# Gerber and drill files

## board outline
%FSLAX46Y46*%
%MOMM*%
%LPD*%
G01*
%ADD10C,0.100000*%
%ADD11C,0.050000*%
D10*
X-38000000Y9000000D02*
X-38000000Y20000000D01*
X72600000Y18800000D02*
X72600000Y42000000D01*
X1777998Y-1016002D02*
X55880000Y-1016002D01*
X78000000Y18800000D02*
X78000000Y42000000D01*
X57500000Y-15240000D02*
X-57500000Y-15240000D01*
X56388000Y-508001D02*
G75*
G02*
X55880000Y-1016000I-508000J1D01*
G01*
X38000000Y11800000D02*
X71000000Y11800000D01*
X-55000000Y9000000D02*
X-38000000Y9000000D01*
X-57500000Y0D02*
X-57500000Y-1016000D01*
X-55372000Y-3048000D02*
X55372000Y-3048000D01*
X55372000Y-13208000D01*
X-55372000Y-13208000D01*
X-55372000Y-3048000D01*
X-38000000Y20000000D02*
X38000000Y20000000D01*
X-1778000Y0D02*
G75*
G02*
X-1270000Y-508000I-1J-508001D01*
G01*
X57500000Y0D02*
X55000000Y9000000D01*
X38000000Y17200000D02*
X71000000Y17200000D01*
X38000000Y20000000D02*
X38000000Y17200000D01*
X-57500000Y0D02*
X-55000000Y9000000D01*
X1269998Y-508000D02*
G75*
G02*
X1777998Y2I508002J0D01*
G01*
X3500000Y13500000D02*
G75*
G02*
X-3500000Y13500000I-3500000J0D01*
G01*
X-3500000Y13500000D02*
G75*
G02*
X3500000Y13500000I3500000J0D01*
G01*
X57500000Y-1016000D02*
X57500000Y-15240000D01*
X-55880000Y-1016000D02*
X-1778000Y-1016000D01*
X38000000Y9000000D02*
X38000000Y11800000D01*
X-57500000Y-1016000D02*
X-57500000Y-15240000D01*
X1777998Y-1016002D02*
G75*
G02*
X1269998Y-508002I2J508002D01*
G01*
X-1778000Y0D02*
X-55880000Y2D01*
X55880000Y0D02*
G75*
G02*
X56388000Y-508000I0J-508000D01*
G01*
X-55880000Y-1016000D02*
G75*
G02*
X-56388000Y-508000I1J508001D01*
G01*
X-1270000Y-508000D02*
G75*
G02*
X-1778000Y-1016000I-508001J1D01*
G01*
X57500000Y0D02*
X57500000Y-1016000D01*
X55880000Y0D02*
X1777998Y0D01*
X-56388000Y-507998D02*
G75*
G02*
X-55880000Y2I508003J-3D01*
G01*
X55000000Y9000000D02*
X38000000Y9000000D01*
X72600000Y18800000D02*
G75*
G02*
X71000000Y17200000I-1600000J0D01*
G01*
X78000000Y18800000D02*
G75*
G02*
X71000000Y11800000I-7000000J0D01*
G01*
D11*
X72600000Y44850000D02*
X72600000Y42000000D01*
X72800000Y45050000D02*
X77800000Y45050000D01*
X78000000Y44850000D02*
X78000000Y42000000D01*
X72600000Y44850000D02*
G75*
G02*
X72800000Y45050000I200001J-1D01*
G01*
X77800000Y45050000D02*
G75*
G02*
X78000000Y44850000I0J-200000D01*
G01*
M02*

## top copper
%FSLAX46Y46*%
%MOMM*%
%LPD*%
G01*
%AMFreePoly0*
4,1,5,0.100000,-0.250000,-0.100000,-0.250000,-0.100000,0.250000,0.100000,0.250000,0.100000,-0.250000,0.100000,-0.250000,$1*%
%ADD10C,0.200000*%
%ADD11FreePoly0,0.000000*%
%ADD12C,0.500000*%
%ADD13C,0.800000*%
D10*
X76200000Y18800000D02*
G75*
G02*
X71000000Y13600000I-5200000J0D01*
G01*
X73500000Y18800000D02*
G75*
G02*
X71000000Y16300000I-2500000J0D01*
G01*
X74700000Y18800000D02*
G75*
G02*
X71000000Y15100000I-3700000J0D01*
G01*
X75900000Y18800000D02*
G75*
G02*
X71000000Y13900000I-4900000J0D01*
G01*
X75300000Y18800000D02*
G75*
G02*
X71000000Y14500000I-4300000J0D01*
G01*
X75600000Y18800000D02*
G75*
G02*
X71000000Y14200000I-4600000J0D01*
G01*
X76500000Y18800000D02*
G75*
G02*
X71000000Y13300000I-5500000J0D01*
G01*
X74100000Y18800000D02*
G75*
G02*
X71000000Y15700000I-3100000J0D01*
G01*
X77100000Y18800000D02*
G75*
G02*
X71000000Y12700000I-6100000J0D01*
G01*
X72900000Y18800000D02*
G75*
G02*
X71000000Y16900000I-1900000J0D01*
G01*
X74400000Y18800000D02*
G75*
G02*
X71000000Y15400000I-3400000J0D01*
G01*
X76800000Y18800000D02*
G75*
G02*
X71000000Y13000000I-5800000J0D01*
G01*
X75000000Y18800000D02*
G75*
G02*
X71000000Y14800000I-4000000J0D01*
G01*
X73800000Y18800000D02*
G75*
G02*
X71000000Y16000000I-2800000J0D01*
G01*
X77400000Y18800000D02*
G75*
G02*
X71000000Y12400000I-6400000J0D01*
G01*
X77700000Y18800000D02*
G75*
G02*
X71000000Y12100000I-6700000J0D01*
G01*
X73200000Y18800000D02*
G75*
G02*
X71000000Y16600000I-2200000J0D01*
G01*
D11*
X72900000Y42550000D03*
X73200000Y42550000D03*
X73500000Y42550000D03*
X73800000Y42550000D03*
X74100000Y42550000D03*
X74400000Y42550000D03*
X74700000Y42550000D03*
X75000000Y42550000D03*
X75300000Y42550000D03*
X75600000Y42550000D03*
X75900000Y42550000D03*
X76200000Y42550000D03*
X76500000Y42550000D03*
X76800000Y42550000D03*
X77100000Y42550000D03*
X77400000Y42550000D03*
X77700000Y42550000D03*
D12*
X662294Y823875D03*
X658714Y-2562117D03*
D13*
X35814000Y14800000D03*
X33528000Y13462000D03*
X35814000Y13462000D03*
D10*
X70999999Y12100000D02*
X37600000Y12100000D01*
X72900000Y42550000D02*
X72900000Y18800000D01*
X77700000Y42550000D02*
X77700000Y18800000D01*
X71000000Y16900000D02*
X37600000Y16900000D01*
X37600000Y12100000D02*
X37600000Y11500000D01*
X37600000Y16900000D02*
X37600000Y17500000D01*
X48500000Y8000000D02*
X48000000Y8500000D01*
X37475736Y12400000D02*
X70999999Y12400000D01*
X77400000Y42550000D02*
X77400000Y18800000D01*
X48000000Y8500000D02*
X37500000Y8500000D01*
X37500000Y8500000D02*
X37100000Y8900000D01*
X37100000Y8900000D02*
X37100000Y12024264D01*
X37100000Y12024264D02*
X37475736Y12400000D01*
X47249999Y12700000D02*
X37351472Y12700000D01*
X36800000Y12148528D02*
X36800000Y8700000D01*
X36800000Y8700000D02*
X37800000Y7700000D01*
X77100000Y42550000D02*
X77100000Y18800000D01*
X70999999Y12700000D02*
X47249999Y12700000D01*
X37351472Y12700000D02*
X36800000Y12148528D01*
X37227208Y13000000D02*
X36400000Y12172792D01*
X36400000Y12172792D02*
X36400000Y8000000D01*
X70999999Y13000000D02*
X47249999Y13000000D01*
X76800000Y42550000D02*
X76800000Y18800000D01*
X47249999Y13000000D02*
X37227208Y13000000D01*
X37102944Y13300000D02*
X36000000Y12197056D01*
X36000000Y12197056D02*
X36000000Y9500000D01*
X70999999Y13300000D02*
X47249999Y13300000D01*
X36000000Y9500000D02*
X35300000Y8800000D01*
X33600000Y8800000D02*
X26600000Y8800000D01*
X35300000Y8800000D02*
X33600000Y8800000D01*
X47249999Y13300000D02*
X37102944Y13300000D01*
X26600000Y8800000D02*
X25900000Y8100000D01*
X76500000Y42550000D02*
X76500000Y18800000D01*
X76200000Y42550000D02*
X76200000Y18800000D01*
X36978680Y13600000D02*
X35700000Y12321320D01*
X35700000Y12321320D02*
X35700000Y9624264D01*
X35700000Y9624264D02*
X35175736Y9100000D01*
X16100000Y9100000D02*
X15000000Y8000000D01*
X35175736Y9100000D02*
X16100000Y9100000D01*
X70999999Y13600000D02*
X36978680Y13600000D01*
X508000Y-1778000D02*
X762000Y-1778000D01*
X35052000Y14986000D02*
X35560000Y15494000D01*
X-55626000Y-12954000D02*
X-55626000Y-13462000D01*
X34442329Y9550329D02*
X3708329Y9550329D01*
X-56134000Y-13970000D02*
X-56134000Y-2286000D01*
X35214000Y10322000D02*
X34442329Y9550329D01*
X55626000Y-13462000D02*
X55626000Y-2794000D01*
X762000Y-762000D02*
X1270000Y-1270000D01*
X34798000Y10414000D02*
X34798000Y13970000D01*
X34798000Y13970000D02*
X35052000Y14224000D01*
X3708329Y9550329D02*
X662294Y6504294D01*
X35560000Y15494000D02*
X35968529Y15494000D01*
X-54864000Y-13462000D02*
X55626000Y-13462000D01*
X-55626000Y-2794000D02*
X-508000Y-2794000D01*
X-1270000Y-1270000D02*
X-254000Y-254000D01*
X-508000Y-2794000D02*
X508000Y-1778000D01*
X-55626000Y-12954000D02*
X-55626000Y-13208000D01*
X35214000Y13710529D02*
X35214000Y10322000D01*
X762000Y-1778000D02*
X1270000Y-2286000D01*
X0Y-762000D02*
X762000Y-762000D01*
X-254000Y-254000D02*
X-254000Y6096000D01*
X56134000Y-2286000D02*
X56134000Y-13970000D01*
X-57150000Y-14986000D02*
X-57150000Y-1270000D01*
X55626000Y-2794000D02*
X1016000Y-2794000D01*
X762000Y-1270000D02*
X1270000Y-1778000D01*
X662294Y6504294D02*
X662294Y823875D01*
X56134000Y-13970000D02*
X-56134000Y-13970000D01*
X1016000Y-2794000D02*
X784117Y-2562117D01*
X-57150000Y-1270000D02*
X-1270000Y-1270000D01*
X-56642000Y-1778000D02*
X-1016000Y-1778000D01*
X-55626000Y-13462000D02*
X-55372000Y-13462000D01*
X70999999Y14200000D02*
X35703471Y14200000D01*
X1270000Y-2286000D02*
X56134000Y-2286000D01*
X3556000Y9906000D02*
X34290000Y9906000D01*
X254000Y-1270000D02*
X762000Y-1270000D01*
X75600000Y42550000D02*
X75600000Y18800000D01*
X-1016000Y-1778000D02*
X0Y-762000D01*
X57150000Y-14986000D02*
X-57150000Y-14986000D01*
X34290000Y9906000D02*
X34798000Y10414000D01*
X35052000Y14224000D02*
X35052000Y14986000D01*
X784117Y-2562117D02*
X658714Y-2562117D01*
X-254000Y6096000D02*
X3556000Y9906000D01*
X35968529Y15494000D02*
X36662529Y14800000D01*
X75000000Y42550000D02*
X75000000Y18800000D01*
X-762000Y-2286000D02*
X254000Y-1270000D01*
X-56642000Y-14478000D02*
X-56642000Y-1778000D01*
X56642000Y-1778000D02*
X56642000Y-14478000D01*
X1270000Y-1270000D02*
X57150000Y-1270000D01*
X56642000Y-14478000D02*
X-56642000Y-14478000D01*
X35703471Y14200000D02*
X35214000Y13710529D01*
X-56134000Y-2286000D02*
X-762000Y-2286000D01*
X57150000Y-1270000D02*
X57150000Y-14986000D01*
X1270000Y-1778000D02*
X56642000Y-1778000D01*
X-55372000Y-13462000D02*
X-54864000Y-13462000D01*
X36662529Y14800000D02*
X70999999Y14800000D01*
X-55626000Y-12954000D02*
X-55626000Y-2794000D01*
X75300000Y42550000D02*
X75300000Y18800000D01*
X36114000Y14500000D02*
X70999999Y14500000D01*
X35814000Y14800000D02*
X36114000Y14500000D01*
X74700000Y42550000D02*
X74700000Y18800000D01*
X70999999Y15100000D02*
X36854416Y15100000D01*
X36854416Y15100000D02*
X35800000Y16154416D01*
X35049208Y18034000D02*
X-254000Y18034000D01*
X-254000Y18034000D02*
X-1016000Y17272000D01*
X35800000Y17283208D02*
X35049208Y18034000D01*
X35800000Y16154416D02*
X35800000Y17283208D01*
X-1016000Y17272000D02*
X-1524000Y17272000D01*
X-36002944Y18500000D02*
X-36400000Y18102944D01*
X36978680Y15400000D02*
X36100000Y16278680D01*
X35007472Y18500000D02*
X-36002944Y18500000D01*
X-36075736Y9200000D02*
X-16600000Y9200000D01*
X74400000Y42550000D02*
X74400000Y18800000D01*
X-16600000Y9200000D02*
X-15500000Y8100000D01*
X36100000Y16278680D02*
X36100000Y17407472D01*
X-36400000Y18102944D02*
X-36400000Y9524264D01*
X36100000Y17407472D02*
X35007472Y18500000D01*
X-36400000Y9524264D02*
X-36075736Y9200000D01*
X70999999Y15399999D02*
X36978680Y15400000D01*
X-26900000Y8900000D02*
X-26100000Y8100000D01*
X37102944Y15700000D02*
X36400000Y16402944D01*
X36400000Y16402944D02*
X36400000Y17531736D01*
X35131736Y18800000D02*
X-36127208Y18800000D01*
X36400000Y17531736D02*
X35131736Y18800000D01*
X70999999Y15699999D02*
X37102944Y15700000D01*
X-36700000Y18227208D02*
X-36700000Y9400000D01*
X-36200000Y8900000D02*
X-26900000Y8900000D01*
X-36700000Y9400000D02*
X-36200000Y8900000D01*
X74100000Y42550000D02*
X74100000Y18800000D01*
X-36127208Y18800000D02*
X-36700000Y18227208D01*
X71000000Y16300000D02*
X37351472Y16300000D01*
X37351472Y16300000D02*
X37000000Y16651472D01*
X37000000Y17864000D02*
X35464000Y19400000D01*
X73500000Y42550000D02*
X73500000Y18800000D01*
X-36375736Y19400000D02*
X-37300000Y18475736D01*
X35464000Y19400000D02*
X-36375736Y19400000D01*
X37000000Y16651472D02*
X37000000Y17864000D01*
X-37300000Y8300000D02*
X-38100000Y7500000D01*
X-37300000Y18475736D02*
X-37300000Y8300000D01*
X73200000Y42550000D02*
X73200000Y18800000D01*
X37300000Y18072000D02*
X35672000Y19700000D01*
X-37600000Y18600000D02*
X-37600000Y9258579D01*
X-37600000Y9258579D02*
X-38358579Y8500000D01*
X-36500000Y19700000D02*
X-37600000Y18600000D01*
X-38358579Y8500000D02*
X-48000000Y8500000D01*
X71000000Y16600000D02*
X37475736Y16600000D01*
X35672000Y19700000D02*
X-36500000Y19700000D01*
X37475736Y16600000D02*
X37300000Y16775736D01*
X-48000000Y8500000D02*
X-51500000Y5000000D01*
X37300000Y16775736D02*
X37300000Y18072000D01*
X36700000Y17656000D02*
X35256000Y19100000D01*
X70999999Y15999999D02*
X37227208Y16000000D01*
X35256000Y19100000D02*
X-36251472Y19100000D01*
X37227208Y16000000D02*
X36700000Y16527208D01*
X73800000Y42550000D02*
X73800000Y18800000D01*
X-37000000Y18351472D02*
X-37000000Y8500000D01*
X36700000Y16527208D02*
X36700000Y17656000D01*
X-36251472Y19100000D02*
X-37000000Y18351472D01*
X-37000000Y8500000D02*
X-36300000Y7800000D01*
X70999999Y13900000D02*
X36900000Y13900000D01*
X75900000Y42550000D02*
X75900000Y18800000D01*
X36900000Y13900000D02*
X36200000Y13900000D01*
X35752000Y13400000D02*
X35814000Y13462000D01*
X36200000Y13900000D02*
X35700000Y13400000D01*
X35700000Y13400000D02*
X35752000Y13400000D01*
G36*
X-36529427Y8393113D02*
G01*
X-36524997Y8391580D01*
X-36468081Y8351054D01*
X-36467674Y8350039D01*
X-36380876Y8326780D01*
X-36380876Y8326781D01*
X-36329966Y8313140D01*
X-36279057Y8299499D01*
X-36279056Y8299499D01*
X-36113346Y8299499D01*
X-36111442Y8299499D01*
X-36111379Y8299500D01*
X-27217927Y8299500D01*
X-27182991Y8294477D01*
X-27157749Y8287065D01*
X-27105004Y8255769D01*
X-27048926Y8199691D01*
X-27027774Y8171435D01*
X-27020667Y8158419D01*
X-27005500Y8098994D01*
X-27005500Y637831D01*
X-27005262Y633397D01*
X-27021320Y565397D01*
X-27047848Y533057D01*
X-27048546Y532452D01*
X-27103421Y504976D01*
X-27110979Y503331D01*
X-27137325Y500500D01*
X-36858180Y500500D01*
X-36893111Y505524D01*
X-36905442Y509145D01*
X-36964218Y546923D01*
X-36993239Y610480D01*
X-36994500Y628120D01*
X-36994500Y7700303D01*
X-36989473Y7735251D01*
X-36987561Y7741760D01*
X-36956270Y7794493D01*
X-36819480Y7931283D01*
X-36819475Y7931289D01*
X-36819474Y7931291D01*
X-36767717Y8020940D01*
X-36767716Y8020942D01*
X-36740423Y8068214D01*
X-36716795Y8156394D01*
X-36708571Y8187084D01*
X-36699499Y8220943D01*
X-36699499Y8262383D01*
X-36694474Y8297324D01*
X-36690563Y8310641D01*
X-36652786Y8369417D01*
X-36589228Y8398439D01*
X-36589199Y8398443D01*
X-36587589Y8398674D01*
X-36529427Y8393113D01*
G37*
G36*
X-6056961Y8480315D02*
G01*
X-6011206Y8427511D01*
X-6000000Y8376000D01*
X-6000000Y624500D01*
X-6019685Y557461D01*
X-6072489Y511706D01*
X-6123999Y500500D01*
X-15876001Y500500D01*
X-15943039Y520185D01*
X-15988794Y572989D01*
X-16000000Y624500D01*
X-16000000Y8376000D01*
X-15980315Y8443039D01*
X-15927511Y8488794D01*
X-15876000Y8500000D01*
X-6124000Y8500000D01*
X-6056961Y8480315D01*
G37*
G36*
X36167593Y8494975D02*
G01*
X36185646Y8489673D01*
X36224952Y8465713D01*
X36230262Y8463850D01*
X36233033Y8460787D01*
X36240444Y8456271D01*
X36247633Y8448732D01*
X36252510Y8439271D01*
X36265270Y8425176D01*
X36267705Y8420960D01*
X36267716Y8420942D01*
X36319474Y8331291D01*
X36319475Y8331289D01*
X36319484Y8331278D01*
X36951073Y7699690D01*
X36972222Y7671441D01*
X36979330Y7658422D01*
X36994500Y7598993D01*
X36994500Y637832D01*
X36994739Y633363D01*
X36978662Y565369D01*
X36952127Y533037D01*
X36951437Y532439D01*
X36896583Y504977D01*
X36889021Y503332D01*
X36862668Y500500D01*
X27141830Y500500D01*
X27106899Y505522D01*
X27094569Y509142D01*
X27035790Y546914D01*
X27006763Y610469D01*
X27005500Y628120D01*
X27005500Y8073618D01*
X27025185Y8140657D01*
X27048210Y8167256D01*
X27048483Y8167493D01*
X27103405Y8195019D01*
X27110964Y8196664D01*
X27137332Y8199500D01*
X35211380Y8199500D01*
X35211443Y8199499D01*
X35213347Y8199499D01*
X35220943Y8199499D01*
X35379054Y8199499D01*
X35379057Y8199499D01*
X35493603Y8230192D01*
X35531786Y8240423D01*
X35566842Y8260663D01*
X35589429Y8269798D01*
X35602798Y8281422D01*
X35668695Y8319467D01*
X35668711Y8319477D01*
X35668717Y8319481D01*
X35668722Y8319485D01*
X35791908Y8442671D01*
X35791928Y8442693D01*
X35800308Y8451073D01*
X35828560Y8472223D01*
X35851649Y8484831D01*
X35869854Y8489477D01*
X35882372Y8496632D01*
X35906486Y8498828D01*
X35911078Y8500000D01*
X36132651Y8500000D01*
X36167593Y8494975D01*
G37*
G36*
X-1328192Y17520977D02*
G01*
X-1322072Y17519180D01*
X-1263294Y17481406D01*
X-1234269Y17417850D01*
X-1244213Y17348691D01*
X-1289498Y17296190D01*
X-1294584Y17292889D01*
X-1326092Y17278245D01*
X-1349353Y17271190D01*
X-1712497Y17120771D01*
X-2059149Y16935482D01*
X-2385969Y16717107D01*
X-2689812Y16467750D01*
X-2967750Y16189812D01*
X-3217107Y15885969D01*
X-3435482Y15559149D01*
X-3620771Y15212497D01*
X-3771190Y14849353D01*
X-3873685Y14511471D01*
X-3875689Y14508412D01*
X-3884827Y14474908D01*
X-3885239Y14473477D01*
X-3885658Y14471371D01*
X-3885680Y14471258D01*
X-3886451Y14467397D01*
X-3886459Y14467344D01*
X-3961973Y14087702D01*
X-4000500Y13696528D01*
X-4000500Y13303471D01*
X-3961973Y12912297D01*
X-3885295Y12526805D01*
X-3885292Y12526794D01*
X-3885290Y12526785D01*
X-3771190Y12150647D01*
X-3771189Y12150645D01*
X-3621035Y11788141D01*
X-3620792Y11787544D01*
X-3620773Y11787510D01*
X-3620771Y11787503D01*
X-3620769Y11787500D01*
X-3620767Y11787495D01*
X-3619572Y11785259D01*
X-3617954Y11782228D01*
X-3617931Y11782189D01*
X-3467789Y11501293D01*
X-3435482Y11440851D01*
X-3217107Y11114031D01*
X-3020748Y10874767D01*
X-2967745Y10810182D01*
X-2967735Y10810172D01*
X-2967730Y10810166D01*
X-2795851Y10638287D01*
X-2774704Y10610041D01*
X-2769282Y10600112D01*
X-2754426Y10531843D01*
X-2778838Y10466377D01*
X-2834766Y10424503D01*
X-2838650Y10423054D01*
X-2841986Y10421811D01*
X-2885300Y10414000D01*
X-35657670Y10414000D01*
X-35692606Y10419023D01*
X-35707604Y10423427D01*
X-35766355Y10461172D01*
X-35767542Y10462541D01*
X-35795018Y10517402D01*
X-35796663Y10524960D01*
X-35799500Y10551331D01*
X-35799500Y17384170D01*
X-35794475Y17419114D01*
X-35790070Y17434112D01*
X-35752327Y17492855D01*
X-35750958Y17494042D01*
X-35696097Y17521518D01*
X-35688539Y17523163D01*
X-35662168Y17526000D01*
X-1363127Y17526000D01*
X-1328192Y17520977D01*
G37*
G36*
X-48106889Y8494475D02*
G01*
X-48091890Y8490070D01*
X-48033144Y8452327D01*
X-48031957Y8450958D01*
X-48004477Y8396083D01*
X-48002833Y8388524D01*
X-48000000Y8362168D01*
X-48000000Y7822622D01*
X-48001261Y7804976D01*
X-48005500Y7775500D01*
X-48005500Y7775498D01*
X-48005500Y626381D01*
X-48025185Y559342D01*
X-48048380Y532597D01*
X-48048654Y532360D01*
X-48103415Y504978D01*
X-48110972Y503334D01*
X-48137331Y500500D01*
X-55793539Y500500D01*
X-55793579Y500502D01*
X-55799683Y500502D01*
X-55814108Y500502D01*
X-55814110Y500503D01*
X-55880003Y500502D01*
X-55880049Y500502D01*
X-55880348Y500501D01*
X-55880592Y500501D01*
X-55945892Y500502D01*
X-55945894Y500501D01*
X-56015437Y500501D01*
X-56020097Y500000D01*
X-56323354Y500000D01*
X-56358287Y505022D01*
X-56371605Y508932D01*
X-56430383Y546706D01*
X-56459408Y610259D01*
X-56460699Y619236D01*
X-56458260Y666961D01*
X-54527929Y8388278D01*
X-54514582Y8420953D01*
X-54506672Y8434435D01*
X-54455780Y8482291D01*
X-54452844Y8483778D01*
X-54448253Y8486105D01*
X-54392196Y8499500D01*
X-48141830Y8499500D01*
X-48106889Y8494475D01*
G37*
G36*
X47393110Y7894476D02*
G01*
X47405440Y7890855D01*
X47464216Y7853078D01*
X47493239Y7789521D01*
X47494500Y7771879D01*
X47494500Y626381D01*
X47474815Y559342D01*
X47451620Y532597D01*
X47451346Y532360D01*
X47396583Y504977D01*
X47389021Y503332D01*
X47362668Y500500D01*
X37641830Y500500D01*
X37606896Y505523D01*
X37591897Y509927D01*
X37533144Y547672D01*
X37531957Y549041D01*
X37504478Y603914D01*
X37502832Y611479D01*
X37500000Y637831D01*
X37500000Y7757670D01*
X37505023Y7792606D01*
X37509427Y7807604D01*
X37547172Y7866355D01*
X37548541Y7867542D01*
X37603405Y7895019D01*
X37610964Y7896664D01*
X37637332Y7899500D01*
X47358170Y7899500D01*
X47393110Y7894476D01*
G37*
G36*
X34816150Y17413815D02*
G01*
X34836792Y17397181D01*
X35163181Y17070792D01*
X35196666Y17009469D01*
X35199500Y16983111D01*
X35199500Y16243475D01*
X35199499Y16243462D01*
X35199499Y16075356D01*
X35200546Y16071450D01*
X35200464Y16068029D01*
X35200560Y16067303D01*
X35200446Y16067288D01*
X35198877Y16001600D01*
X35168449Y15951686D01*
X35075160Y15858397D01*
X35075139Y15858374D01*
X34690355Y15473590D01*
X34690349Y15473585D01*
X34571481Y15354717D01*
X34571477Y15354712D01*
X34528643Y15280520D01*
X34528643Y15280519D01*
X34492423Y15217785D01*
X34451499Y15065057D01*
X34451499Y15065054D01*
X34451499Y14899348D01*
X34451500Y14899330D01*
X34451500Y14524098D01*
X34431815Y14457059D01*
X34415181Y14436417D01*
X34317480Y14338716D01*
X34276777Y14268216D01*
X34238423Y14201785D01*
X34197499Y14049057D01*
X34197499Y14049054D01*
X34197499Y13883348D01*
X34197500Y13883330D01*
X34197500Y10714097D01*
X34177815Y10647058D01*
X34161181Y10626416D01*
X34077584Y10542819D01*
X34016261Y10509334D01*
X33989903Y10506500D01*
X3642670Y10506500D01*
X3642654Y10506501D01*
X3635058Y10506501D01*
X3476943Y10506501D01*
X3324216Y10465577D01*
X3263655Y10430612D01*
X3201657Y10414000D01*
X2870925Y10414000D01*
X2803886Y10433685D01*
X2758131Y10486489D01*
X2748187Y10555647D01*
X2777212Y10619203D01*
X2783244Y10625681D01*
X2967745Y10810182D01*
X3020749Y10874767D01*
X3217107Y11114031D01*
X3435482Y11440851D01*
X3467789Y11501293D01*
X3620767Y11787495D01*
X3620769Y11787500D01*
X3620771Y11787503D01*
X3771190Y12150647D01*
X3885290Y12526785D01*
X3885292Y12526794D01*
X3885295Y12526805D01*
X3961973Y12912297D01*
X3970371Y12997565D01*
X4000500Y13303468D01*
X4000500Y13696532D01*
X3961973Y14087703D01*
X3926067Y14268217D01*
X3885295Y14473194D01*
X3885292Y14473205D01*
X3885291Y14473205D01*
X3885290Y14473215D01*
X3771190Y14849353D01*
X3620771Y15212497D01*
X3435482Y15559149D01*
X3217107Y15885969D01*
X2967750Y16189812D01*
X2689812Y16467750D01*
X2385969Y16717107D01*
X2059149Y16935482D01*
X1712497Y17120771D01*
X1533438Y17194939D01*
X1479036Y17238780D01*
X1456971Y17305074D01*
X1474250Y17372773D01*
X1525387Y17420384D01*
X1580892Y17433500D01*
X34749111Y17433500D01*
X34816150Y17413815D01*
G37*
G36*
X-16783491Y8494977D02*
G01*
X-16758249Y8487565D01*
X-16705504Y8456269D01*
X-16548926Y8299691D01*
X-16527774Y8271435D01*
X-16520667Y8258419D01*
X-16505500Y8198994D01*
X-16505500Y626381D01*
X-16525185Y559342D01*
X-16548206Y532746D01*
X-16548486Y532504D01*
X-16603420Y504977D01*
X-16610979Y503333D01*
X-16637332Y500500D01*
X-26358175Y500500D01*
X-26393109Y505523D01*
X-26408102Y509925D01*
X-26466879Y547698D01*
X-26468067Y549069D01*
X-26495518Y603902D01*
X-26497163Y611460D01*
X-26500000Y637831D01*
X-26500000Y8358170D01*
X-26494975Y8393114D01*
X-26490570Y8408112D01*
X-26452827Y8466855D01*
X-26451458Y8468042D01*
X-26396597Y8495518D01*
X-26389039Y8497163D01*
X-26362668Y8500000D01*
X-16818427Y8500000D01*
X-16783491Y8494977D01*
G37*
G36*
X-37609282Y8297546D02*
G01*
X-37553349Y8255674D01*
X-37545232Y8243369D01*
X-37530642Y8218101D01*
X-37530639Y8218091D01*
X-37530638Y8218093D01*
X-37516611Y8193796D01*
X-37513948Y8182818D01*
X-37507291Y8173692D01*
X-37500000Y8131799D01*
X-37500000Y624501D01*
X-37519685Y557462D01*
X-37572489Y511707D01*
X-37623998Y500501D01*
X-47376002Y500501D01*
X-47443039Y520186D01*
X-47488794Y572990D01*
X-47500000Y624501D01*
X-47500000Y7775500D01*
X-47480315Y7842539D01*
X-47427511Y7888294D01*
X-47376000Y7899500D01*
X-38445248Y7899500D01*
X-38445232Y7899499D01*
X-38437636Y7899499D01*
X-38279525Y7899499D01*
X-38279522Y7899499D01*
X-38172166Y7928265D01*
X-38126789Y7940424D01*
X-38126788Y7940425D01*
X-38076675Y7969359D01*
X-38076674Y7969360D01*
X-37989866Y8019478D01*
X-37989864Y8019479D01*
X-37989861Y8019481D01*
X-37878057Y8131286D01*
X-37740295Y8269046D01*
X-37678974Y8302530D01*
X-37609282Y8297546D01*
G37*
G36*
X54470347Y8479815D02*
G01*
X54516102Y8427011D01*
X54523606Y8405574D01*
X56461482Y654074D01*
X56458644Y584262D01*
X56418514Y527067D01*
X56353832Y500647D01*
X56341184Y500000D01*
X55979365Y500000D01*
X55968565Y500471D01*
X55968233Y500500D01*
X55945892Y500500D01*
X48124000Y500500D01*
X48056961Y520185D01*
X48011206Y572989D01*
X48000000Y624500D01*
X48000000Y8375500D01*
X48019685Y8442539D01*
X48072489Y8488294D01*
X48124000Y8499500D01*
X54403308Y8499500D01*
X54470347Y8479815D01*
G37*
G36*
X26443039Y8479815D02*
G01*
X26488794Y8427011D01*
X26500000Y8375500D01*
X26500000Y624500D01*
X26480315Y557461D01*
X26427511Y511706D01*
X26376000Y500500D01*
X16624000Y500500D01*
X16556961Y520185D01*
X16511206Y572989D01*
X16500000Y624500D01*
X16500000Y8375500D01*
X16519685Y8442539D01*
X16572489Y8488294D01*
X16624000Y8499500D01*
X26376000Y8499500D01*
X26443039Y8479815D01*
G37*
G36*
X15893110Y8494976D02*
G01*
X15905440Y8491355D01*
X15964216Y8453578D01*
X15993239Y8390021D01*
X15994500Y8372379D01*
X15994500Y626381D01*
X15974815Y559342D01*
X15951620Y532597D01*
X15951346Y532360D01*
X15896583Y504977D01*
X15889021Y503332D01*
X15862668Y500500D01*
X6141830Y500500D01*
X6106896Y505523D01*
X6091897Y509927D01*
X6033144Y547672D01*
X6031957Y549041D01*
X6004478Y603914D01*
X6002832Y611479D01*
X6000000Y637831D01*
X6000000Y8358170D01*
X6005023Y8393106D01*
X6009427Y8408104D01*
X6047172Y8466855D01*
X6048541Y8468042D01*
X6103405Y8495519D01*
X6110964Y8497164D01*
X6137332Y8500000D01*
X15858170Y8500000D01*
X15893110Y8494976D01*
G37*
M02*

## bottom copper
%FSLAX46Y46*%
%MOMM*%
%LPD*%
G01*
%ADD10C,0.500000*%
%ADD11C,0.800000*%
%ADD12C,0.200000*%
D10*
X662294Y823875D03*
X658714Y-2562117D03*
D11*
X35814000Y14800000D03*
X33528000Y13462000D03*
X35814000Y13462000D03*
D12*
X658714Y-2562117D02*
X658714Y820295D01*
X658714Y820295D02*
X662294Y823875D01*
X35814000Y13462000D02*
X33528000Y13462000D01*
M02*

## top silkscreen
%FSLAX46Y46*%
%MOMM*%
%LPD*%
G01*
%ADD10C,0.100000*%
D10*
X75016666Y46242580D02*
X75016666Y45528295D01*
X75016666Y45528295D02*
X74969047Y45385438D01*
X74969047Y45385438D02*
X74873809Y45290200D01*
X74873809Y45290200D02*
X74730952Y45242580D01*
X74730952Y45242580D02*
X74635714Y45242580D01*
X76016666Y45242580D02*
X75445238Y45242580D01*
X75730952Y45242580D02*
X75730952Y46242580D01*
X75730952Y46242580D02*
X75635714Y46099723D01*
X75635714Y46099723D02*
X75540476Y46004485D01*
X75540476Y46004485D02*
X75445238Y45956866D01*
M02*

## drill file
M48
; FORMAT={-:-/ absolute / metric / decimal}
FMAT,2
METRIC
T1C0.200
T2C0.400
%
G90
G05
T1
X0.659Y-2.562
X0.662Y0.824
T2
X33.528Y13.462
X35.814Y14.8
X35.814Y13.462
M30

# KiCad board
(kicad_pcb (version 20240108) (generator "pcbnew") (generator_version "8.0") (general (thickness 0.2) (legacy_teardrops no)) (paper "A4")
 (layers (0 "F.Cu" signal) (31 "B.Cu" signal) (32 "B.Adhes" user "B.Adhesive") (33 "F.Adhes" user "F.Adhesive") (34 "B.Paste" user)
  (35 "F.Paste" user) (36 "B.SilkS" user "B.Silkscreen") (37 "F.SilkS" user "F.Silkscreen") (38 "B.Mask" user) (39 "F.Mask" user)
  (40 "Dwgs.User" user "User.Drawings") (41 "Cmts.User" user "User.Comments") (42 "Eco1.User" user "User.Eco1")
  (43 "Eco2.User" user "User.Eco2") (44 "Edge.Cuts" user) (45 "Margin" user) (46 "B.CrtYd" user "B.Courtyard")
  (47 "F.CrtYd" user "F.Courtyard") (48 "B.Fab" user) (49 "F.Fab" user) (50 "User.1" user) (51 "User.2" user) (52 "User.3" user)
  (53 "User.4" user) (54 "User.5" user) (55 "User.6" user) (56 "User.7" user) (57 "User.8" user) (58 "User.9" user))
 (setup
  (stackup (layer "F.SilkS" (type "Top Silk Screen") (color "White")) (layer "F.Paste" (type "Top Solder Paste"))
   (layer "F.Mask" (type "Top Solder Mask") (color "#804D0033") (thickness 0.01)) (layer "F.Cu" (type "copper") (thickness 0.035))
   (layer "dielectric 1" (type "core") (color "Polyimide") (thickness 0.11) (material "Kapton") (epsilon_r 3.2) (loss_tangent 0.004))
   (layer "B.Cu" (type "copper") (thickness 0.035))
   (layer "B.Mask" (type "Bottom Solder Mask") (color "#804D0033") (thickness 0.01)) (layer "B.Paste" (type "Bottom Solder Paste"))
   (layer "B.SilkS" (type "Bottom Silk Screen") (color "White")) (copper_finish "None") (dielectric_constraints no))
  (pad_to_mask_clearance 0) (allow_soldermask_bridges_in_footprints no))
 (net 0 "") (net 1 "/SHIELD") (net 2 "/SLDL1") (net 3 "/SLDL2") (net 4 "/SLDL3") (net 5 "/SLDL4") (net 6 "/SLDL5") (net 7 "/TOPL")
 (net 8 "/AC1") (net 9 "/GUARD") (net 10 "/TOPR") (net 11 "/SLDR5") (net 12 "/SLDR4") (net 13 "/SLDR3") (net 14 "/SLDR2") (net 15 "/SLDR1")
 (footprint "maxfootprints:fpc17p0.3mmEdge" (layer "F.Cu") (at 75.3 -45.05)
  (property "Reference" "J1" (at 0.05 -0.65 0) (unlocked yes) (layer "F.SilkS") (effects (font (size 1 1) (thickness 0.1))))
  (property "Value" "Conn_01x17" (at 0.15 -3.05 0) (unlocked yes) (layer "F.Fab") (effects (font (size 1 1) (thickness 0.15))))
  (fp_line (start -2.7 0.2) (end -2.7 3.05) (stroke (width 0.05) (type default)) (layer "Edge.Cuts"))
  (fp_line (start -2.5 0) (end 2.5 0) (stroke (width 0.05) (type default)) (layer "Edge.Cuts"))
  (fp_line (start 2.7 0.2) (end 2.7 3.05) (stroke (width 0.05) (type default)) (layer "Edge.Cuts"))
  (fp_arc (start -2.7 0.2) (mid -2.641421 0.058579) (end -2.5 0) (stroke (width 0.05) (type default)) (layer "Edge.Cuts"))
  (fp_arc (start 2.5 0) (mid 2.641421 0.058579) (end 2.7 0.2) (stroke (width 0.05) (type default)) (layer "Edge.Cuts"))
  (pad "1" connect custom (at -2.4 2.5) (size 0.2 0.5) (layers "F.Cu") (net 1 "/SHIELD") (options (clearance outline) (anchor rect))
   (primitives))
  (pad "2" connect custom (at -2.1 2.5) (size 0.2 0.5) (layers "F.Cu") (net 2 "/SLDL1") (options (clearance outline) (anchor rect))
   (primitives))
  (pad "3" connect custom (at -1.8 2.5) (size 0.2 0.5) (layers "F.Cu") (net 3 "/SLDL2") (options (clearance outline) (anchor rect))
   (primitives))
  (pad "4" connect custom (at -1.5 2.5) (size 0.2 0.5) (layers "F.Cu") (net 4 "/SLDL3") (options (clearance outline) (anchor rect))
   (primitives))
  (pad "5" connect custom (at -1.2 2.5) (size 0.2 0.5) (layers "F.Cu") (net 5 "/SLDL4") (options (clearance outline) (anchor rect))
   (primitives))
  (pad "6" connect custom (at -0.9 2.5) (size 0.2 0.5) (layers "F.Cu") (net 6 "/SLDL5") (options (clearance outline) (anchor rect))
   (primitives))
  (pad "7" connect custom (at -0.6 2.5) (size 0.2 0.5) (layers "F.Cu") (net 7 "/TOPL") (options (clearance outline) (anchor rect))
   (primitives))
  (pad "8" connect custom (at -0.3 2.5) (size 0.2 0.5) (layers "F.Cu") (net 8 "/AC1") (options (clearance outline) (anchor rect))
   (primitives))
  (pad "9" connect custom (at 0 2.5) (size 0.2 0.5) (layers "F.Cu") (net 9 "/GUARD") (options (clearance outline) (anchor rect))
   (primitives))
  (pad "10" connect custom (at 0.3 2.5) (size 0.2 0.5) (layers "F.Cu") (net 8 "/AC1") (options (clearance outline) (anchor rect))
   (primitives))
  (pad "11" connect custom (at 0.6 2.5) (size 0.2 0.5) (layers "F.Cu") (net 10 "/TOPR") (options (clearance outline) (anchor rect))
   (primitives))
  (pad "12" connect custom (at 0.9 2.5) (size 0.2 0.5) (layers "F.Cu") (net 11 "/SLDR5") (options (clearance outline) (anchor rect))
   (primitives))
  (pad "13" connect custom (at 1.2 2.5) (size 0.2 0.5) (layers "F.Cu") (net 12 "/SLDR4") (options (clearance outline) (anchor rect))
   (primitives))
  (pad "14" connect custom (at 1.5 2.5) (size 0.2 0.5) (layers "F.Cu") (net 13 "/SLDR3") (options (clearance outline) (anchor rect))
   (primitives))
  (pad "15" connect custom (at 1.8 2.5) (size 0.2 0.5) (layers "F.Cu") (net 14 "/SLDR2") (options (clearance outline) (anchor rect))
   (primitives))
  (pad "16" connect custom (at 2.1 2.5) (size 0.2 0.5) (layers "F.Cu") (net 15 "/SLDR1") (options (clearance outline) (anchor rect))
   (primitives))
  (pad "17" connect custom (at 2.4 2.5) (size 0.2 0.5) (layers "F.Cu") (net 1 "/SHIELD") (options (clearance outline) (anchor rect))
   (primitives)))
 (gr_arc (start 76.2 -18.8) (mid 74.676955 -15.123045) (end 71 -13.6) (stroke (width 0.2) (type default)) (layer "F.Cu") (net 11))
 (gr_arc (start 73.5 -18.8) (mid 72.767767 -17.032233) (end 71 -16.3) (stroke (width 0.2) (type default)) (layer "F.Cu") (net 3))
 (gr_arc (start 74.7 -18.8) (mid 73.616295 -16.183705) (end 71 -15.1) (stroke (width 0.2) (type default)) (layer "F.Cu") (net 7))
 (gr_arc (start 75.9 -18.8) (mid 74.464823 -15.335177) (end 71 -13.9) (stroke (width 0.2) (type default)) (layer "F.Cu") (net 10))
 (gr_arc (start 75.3 -18.8) (mid 74.040559 -15.759441) (end 71 -14.5) (stroke (width 0.2) (type default)) (layer "F.Cu") (net 9))
 (gr_arc (start 75.6 -18.8) (mid 74.252691 -15.547309) (end 71 -14.2) (stroke (width 0.2) (type default)) (layer "F.Cu") (net 8))
 (gr_arc (start 76.5 -18.8) (mid 74.889087 -14.910913) (end 71 -13.3) (stroke (width 0.2) (type default)) (layer "F.Cu") (net 12))
 (gr_arc (start 74.1 -18.8) (mid 73.192031 -16.607969) (end 71 -15.7) (stroke (width 0.2) (type default)) (layer "F.Cu") (net 5))
 (gr_arc (start 77.1 -18.8) (mid 75.313351 -14.486649) (end 71 -12.7) (stroke (width 0.2) (type default)) (layer "F.Cu") (net 14))
 (gr_arc (start 72.9 -18.8) (mid 72.343503 -17.456497) (end 71 -16.9) (stroke (width 0.2) (type default)) (layer "F.Cu") (net 1))
 (gr_arc (start 74.4 -18.8) (mid 73.404163 -16.395837) (end 71 -15.4) (stroke (width 0.2) (type default)) (layer "F.Cu") (net 6))
 (gr_arc (start 76.8 -18.8) (mid 75.101219 -14.698781) (end 71 -13) (stroke (width 0.2) (type default)) (layer "F.Cu") (net 13))
 (gr_arc (start 75 -18.8) (mid 73.828427 -15.971573) (end 71 -14.8) (stroke (width 0.2) (type default)) (layer "F.Cu") (net 8))
 (gr_arc (start 73.8 -18.8) (mid 72.979899 -16.820101) (end 71 -16) (stroke (width 0.2) (type default)) (layer "F.Cu") (net 4))
 (gr_arc (start 77.4 -18.8) (mid 75.525483 -14.274517) (end 71 -12.4) (stroke (width 0.2) (type default)) (layer "F.Cu") (net 15))
 (gr_arc (start 77.7 -18.8) (mid 75.737615 -14.062385) (end 71 -12.1) (stroke (width 0.2) (type default)) (layer "F.Cu") (net 1))
 (gr_arc (start 73.2 -18.8) (mid 72.555635 -17.244365) (end 71 -16.6) (stroke (width 0.2) (type default)) (layer "F.Cu") (net 2))
 (gr_line (start -38 -9) (end -38 -20) (stroke (width 0.1) (type default)) (layer "Edge.Cuts"))
 (gr_line (start 72.6 -18.8) (end 72.6 -42) (stroke (width 0.1) (type default)) (layer "Edge.Cuts"))
 (gr_line (start 1.777998 1.016002) (end 55.88 1.016002) (stroke (width 0.1) (type default)) (layer "Edge.Cuts"))
 (gr_line (start 78 -18.8) (end 78 -42) (stroke (width 0.1) (type default)) (layer "Edge.Cuts"))
 (gr_line (start 57.5 15.24) (end -57.5 15.24) (stroke (width 0.1) (type default)) (layer "Edge.Cuts"))
 (gr_arc (start 56.388 0.508001) (mid 56.23921 0.867211) (end 55.88 1.016002) (stroke (width 0.1) (type default)) (layer "Edge.Cuts"))
 (gr_line (start 38 -11.8) (end 71 -11.8) (stroke (width 0.1) (type default)) (layer "Edge.Cuts"))
 (gr_line (start -55 -9) (end -38 -9) (stroke (width 0.1) (type default)) (layer "Edge.Cuts"))
 (gr_line (start -57.5 0) (end -57.5 1.016) (stroke (width 0.1) (type default)) (layer "Edge.Cuts"))
 (gr_rect (start -55.372 3.048) (end 55.372 13.208) (stroke (width 0.1) (type default)) (fill none) (layer "Edge.Cuts"))
 (gr_line (start -38 -20) (end 38 -20) (stroke (width 0.1) (type default)) (layer "Edge.Cuts"))
 (gr_arc (start -1.778 0) (mid -1.41879 0.14879) (end -1.27 0.508) (stroke (width 0.1) (type default)) (layer "Edge.Cuts"))
 (gr_line (start 57.5 0) (end 55 -9) (stroke (width 0.1) (type default)) (layer "Edge.Cuts"))
 (gr_line (start 38 -17.2) (end 71 -17.2) (stroke (width 0.1) (type default)) (layer "Edge.Cuts"))
 (gr_line (start 38 -20) (end 38 -17.2) (stroke (width 0.1) (type default)) (layer "Edge.Cuts"))
 (gr_line (start -57.5 0) (end -55 -9) (stroke (width 0.1) (type default)) (layer "Edge.Cuts"))
 (gr_arc (start 1.269998 0.508) (mid 1.418788 0.14879) (end 1.777998 0) (stroke (width 0.1) (type default)) (layer "Edge.Cuts"))
 (gr_circle (center 0 -13.5) (end 0 -10) (stroke (width 0.1) (type default)) (fill none) (layer "Edge.Cuts"))
 (gr_line (start 57.5 1.016) (end 57.5 15.24) (stroke (width 0.1) (type default)) (layer "Edge.Cuts"))
 (gr_line (start -55.88 1.016) (end -1.778 1.016) (stroke (width 0.1) (type default)) (layer "Edge.Cuts"))
 (gr_line (start 38 -9) (end 38 -11.8) (stroke (width 0.1) (type default)) (layer "Edge.Cuts"))
 (gr_line (start -57.5 1.016) (end -57.5 15.24) (stroke (width 0.1) (type default)) (layer "Edge.Cuts"))
 (gr_arc (start 1.777998 1.016002) (mid 1.418788 0.867212) (end 1.269998 0.508002) (stroke (width 0.1) (type default)) (layer "Edge.Cuts"))
 (gr_line (start -1.778 0) (end -55.88 -0.000002) (stroke (width 0.1) (type default)) (layer "Edge.Cuts"))
 (gr_arc (start 55.88 0) (mid 56.23921 0.14879) (end 56.388 0.508) (stroke (width 0.1) (type default)) (layer "Edge.Cuts"))
 (gr_arc (start -55.88 1.016) (mid -56.23921 0.86721) (end -56.388 0.508) (stroke (width 0.1) (type default)) (layer "Edge.Cuts"))
 (gr_arc (start -1.27 0.508) (mid -1.41879 0.86721) (end -1.778 1.016) (stroke (width 0.1) (type default)) (layer "Edge.Cuts"))
 (gr_line (start 57.5 0) (end 57.5 1.016) (stroke (width 0.1) (type default)) (layer "Edge.Cuts"))
 (gr_line (start 55.88 0) (end 1.777998 0) (stroke (width 0.1) (type default)) (layer "Edge.Cuts"))
 (gr_arc (start -56.388 0.507998) (mid -56.23921 0.148789) (end -55.88 -0.000002) (stroke (width 0.1) (type default)) (layer "Edge.Cuts"))
 (gr_line (start 55 -9) (end 38 -9) (stroke (width 0.1) (type default)) (layer "Edge.Cuts"))
 (gr_arc (start 72.6 -18.8) (mid 72.131371 -17.668629) (end 71 -17.2) (stroke (width 0.1) (type default)) (layer "Edge.Cuts"))
 (gr_arc (start 78 -18.8) (mid 75.949747 -13.850253) (end 71 -11.8) (stroke (width 0.1) (type default)) (layer "Edge.Cuts"))
 (segment (start 70.999999 -12.1) (end 37.6 -12.1) (width 0.2) (layer "F.Cu") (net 1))
 (segment (start 72.9 -42.55) (end 72.9 -18.8) (width 0.2) (layer "F.Cu") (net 1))
 (segment (start 77.7 -42.55) (end 77.7 -18.8) (width 0.2) (layer "F.Cu") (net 1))
 (segment (start 71 -16.9) (end 37.6 -16.9) (width 0.2) (layer "F.Cu") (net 1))
 (segment (start 37.6 -12.1) (end 37.6 -11.5) (width 0.2) (layer "F.Cu") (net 1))
 (segment (start 37.6 -16.9) (end 37.6 -17.5) (width 0.2) (layer "F.Cu") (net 1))
 (segment (start 48.5 -8) (end 48 -8.5) (width 0.2) (layer "F.Cu") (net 15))
 (segment (start 37.475736 -12.4) (end 70.999999 -12.4) (width 0.2) (layer "F.Cu") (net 15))
 (segment (start 77.4 -42.55) (end 77.4 -18.8) (width 0.2) (layer "F.Cu") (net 15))
 (segment (start 48 -8.5) (end 37.5 -8.5) (width 0.2) (layer "F.Cu") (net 15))
 (segment (start 37.5 -8.5) (end 37.1 -8.9) (width 0.2) (layer "F.Cu") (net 15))
 (segment (start 37.1 -8.9) (end 37.1 -12.024264) (width 0.2) (layer "F.Cu") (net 15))
 (segment (start 37.1 -12.024264) (end 37.475736 -12.4) (width 0.2) (layer "F.Cu") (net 15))
 (segment (start 47.249999 -12.7) (end 37.351472 -12.7) (width 0.2) (layer "F.Cu") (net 14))
 (segment (start 36.8 -12.148528) (end 36.8 -8.7) (width 0.2) (layer "F.Cu") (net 14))
 (segment (start 36.8 -8.7) (end 37.8 -7.7) (width 0.2) (layer "F.Cu") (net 14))
 (segment (start 77.1 -42.55) (end 77.1 -18.8) (width 0.2) (layer "F.Cu") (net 14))
 (segment (start 70.999999 -12.7) (end 47.249999 -12.7) (width 0.2) (layer "F.Cu") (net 14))
 (segment (start 37.351472 -12.7) (end 36.8 -12.148528) (width 0.2) (layer "F.Cu") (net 14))
 (segment (start 37.227208 -13) (end 36.4 -12.172792) (width 0.2) (layer "F.Cu") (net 13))
 (segment (start 36.4 -12.172792) (end 36.4 -8) (width 0.2) (layer "F.Cu") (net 13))
 (segment (start 70.999999 -13) (end 47.249999 -13) (width 0.2) (layer "F.Cu") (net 13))
 (segment (start 76.8 -42.55) (end 76.8 -18.8) (width 0.2) (layer "F.Cu") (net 13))
 (segment (start 47.249999 -13) (end 37.227208 -13) (width 0.2) (layer "F.Cu") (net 13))
 (segment (start 37.102944 -13.3) (end 36 -12.197056) (width 0.2) (layer "F.Cu") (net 12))
 (segment (start 36 -12.197056) (end 36 -9.5) (width 0.2) (layer "F.Cu") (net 12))
 (segment (start 70.999999 -13.3) (end 47.249999 -13.3) (width 0.2) (layer "F.Cu") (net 12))
 (segment (start 36 -9.5) (end 35.3 -8.8) (width 0.2) (layer "F.Cu") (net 12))
 (segment (start 33.6 -8.8) (end 26.6 -8.8) (width 0.2) (layer "F.Cu") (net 12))
 (segment (start 35.3 -8.8) (end 33.6 -8.8) (width 0.2) (layer "F.Cu") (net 12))
 (segment (start 47.249999 -13.3) (end 37.102944 -13.3) (width 0.2) (layer "F.Cu") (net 12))
 (segment (start 26.6 -8.8) (end 25.9 -8.1) (width 0.2) (layer "F.Cu") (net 12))
 (segment (start 76.5 -42.55) (end 76.5 -18.8) (width 0.2) (layer "F.Cu") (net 12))
 (segment (start 76.2 -42.55) (end 76.2 -18.8) (width 0.2) (layer "F.Cu") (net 11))
 (segment (start 36.97868 -13.6) (end 35.7 -12.32132) (width 0.2) (layer "F.Cu") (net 11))
 (segment (start 35.7 -12.32132) (end 35.7 -9.624264) (width 0.2) (layer "F.Cu") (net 11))
 (segment (start 35.7 -9.624264) (end 35.175736 -9.1) (width 0.2) (layer "F.Cu") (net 11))
 (segment (start 16.1 -9.1) (end 15 -8) (width 0.2) (layer "F.Cu") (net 11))
 (segment (start 35.175736 -9.1) (end 16.1 -9.1) (width 0.2) (layer "F.Cu") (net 11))
 (segment (start 70.999999 -13.6) (end 36.97868 -13.6) (width 0.2) (layer "F.Cu") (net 11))
 (segment (start 0.508 1.778) (end 0.762 1.778) (width 0.2) (layer "F.Cu") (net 8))
 (segment (start 35.052 -14.986) (end 35.56 -15.494) (width 0.2) (layer "F.Cu") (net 8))
 (segment (start -55.626 12.954) (end -55.626 13.462) (width 0.2) (layer "F.Cu") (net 8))
 (segment (start 34.442329 -9.550329) (end 3.708329 -9.550329) (width 0.2) (layer "F.Cu") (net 8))
 (segment (start -56.134 13.97) (end -56.134 2.286) (width 0.2) (layer "F.Cu") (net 8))
 (segment (start 35.214 -10.322) (end 34.442329 -9.550329) (width 0.2) (layer "F.Cu") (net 8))
 (segment (start 55.626 13.462) (end 55.626 2.794) (width 0.2) (layer "F.Cu") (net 8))
 (segment (start 0.762 0.762) (end 1.27 1.27) (width 0.2) (layer "F.Cu") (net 8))
 (segment (start 34.798 -10.414) (end 34.798 -13.97) (width 0.2) (layer "F.Cu") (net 8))
 (segment (start 34.798 -13.97) (end 35.052 -14.224) (width 0.2) (layer "F.Cu") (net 8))
 (segment (start 3.708329 -9.550329) (end 0.662294 -6.504294) (width 0.2) (layer "F.Cu") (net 8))
 (segment (start 35.56 -15.494) (end 35.968529 -15.494) (width 0.2) (layer "F.Cu") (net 8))
 (segment (start -54.864 13.462) (end 55.626 13.462) (width 0.2) (layer "F.Cu") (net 8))
 (segment (start -55.626 2.794) (end -0.508 2.794) (width 0.2) (layer "F.Cu") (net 8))
 (segment (start -1.27 1.27) (end -0.254 0.254) (width 0.2) (layer "F.Cu") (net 8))
 (segment (start -0.508 2.794) (end 0.508 1.778) (width 0.2) (layer "F.Cu") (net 8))
 (segment (start -55.626 12.954) (end -55.626 13.208) (width 0.2) (layer "F.Cu") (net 8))
 (segment (start 35.214 -13.710529) (end 35.214 -10.322) (width 0.2) (layer "F.Cu") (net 8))
 (segment (start 0.762 1.778) (end 1.27 2.286) (width 0.2) (layer "F.Cu") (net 8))
 (segment (start 0 0.762) (end 0.762 0.762) (width 0.2) (layer "F.Cu") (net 8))
 (segment (start -0.254 0.254) (end -0.254 -6.096) (width 0.2) (layer "F.Cu") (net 8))
 (segment (start 56.134 2.286) (end 56.134 13.97) (width 0.2) (layer "F.Cu") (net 8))
 (segment (start -57.15 14.986) (end -57.15 1.27) (width 0.2) (layer "F.Cu") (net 8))
 (segment (start 55.626 2.794) (end 1.016 2.794) (width 0.2) (layer "F.Cu") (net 8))
 (segment (start 0.762 1.27) (end 1.27 1.778) (width 0.2) (layer "F.Cu") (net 8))
 (segment (start 0.662294 -6.504294) (end 0.662294 -0.823875) (width 0.2) (layer "F.Cu") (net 8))
 (segment (start 56.134 13.97) (end -56.134 13.97) (width 0.2) (layer "F.Cu") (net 8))
 (segment (start 1.016 2.794) (end 0.784117 2.562117) (width 0.2) (layer "F.Cu") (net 8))
 (segment (start -57.15 1.27) (end -1.27 1.27) (width 0.2) (layer "F.Cu") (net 8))
 (segment (start -56.642 1.778) (end -1.016 1.778) (width 0.2) (layer "F.Cu") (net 8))
 (segment (start -55.626 13.462) (end -55.372 13.462) (width 0.2) (layer "F.Cu") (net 8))
 (segment (start 70.999999 -14.2) (end 35.703471 -14.2) (width 0.2) (layer "F.Cu") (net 8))
 (segment (start 1.27 2.286) (end 56.134 2.286) (width 0.2) (layer "F.Cu") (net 8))
 (segment (start 3.556 -9.906) (end 34.29 -9.906) (width 0.2) (layer "F.Cu") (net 8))
 (segment (start 0.254 1.27) (end 0.762 1.27) (width 0.2) (layer "F.Cu") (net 8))
 (segment (start 75.6 -42.55) (end 75.6 -18.8) (width 0.2) (layer "F.Cu") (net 8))
 (segment (start -1.016 1.778) (end 0 0.762) (width 0.2) (layer "F.Cu") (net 8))
 (segment (start 57.15 14.986) (end -57.15 14.986) (width 0.2) (layer "F.Cu") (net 8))
 (segment (start 34.29 -9.906) (end 34.798 -10.414) (width 0.2) (layer "F.Cu") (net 8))
 (segment (start 35.052 -14.224) (end 35.052 -14.986) (width 0.2) (layer "F.Cu") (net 8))
 (segment (start 0.784117 2.562117) (end 0.658714 2.562117) (width 0.2) (layer "F.Cu") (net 8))
 (segment (start -0.254 -6.096) (end 3.556 -9.906) (width 0.2) (layer "F.Cu") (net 8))
 (segment (start 35.968529 -15.494) (end 36.662529 -14.8) (width 0.2) (layer "F.Cu") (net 8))
 (segment (start 75 -42.55) (end 75 -18.8) (width 0.2) (layer "F.Cu") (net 8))
 (segment (start -0.762 2.286) (end 0.254 1.27) (width 0.2) (layer "F.Cu") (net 8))
 (segment (start -56.642 14.478) (end -56.642 1.778) (width 0.2) (layer "F.Cu") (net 8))
 (segment (start 56.642 1.778) (end 56.642 14.478) (width 0.2) (layer "F.Cu") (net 8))
 (segment (start 1.27 1.27) (end 57.15 1.27) (width 0.2) (layer "F.Cu") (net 8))
 (segment (start 56.642 14.478) (end -56.642 14.478) (width 0.2) (layer "F.Cu") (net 8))
 (segment (start 35.703471 -14.2) (end 35.214 -13.710529) (width 0.2) (layer "F.Cu") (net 8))
 (segment (start -56.134 2.286) (end -0.762 2.286) (width 0.2) (layer "F.Cu") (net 8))
 (segment (start 57.15 1.27) (end 57.15 14.986) (width 0.2) (layer "F.Cu") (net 8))
 (segment (start 1.27 1.778) (end 56.642 1.778) (width 0.2) (layer "F.Cu") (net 8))
 (segment (start -55.372 13.462) (end -54.864 13.462) (width 0.2) (layer "F.Cu") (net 8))
 (segment (start 36.662529 -14.8) (end 70.999999 -14.8) (width 0.2) (layer "F.Cu") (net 8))
 (segment (start -55.626 12.954) (end -55.626 2.794) (width 0.2) (layer "F.Cu") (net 8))
 (via (at 0.662294 -0.823875) (size 0.5) (drill 0.2) (layers "F.Cu" "B.Cu") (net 8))
 (via (at 0.658714 2.562117) (size 0.5) (drill 0.2) (layers "F.Cu" "B.Cu") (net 8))
 (segment (start 0.658714 2.562117) (end 0.658714 -0.820295) (width 0.2) (layer "B.Cu") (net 8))
 (segment (start 0.658714 -0.820295) (end 0.662294 -0.823875) (width 0.2) (layer "B.Cu") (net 8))
 (segment (start 75.3 -42.55) (end 75.3 -18.8) (width 0.2) (layer "F.Cu") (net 9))
 (segment (start 36.114 -14.5) (end 70.999999 -14.5) (width 0.2) (layer "F.Cu") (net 9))
 (segment (start 35.814 -14.8) (end 36.114 -14.5) (width 0.2) (layer "F.Cu") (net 9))
 (via (at 35.814 -14.8) (size 0.8) (drill 0.4) (layers "F.Cu" "B.Cu") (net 9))
 (segment (start 74.7 -42.55) (end 74.7 -18.8) (width 0.2) (layer "F.Cu") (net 7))
 (segment (start 70.999999 -15.1) (end 36.854416 -15.1) (width 0.2) (layer "F.Cu") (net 7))
 (segment (start 36.854416 -15.1) (end 35.8 -16.154416) (width 0.2) (layer "F.Cu") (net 7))
 (segment (start 35.049208 -18.034) (end -0.254 -18.034) (width 0.2) (layer "F.Cu") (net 7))
 (segment (start -0.254 -18.034) (end -1.016 -17.272) (width 0.2) (layer "F.Cu") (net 7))
 (segment (start 35.8 -17.283208) (end 35.049208 -18.034) (width 0.2) (layer "F.Cu") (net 7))
 (segment (start 35.8 -16.154416) (end 35.8 -17.283208) (width 0.2) (layer "F.Cu") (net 7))
 (segment (start -1.016 -17.272) (end -1.524 -17.272) (width 0.2) (layer "F.Cu") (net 7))
 (segment (start -36.002944 -18.5) (end -36.4 -18.102944) (width 0.2) (layer "F.Cu") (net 6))
 (segment (start 36.97868 -15.4) (end 36.1 -16.27868) (width 0.2) (layer "F.Cu") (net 6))
 (segment (start 35.007472 -18.5) (end -36.002944 -18.5) (width 0.2) (layer "F.Cu") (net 6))
 (segment (start -36.075736 -9.2) (end -16.6 -9.2) (width 0.2) (layer "F.Cu") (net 6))
 (segment (start 74.4 -42.55) (end 74.4 -18.8) (width 0.2) (layer "F.Cu") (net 6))
 (segment (start -16.6 -9.2) (end -15.5 -8.1) (width 0.2) (layer "F.Cu") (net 6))
 (segment (start 36.1 -16.27868) (end 36.1 -17.407472) (width 0.2) (layer "F.Cu") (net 6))
 (segment (start -36.4 -18.102944) (end -36.4 -9.524264) (width 0.2) (layer "F.Cu") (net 6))
 (segment (start 36.1 -17.407472) (end 35.007472 -18.5) (width 0.2) (layer "F.Cu") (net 6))
 (segment (start -36.4 -9.524264) (end -36.075736 -9.2) (width 0.2) (layer "F.Cu") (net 6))
 (segment (start 70.999999 -15.399999) (end 36.97868 -15.4) (width 0.2) (layer "F.Cu") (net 6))
 (segment (start -26.9 -8.9) (end -26.1 -8.1) (width 0.2) (layer "F.Cu") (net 5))
 (segment (start 37.102944 -15.7) (end 36.4 -16.402944) (width 0.2) (layer "F.Cu") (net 5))
 (segment (start 36.4 -16.402944) (end 36.4 -17.531736) (width 0.2) (layer "F.Cu") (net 5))
 (segment (start 35.131736 -18.8) (end -36.127208 -18.8) (width 0.2) (layer "F.Cu") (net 5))
 (segment (start 36.4 -17.531736) (end 35.131736 -18.8) (width 0.2) (layer "F.Cu") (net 5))
 (segment (start 70.999999 -15.699999) (end 37.102944 -15.7) (width 0.2) (layer "F.Cu") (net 5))
 (segment (start -36.7 -18.227208) (end -36.7 -9.4) (width 0.2) (layer "F.Cu") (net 5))
 (segment (start -36.2 -8.9) (end -26.9 -8.9) (width 0.2) (layer "F.Cu") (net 5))
 (segment (start -36.7 -9.4) (end -36.2 -8.9) (width 0.2) (layer "F.Cu") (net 5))
 (segment (start 74.1 -42.55) (end 74.1 -18.8) (width 0.2) (layer "F.Cu") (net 5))
 (segment (start -36.127208 -18.8) (end -36.7 -18.227208) (width 0.2) (layer "F.Cu") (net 5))
 (segment (start 71 -16.3) (end 37.351472 -16.3) (width 0.2) (layer "F.Cu") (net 3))
 (segment (start 37.351472 -16.3) (end 37 -16.651472) (width 0.2) (layer "F.Cu") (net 3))
 (segment (start 37 -17.864) (end 35.464 -19.4) (width 0.2) (layer "F.Cu") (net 3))
 (segment (start 73.5 -42.55) (end 73.5 -18.8) (width 0.2) (layer "F.Cu") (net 3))
 (segment (start -36.375736 -19.4) (end -37.3 -18.475736) (width 0.2) (layer "F.Cu") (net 3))
 (segment (start 35.464 -19.4) (end -36.375736 -19.4) (width 0.2) (layer "F.Cu") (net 3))
 (segment (start 37 -16.651472) (end 37 -17.864) (width 0.2) (layer "F.Cu") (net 3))
 (segment (start -37.3 -8.3) (end -38.1 -7.5) (width 0.2) (layer "F.Cu") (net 3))
 (segment (start -37.3 -18.475736) (end -37.3 -8.3) (width 0.2) (layer "F.Cu") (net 3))
 (segment (start 73.2 -42.55) (end 73.2 -18.8) (width 0.2) (layer "F.Cu") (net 2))
 (segment (start 37.3 -18.072) (end 35.672 -19.7) (width 0.2) (layer "F.Cu") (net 2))
 (segment (start -37.6 -18.6) (end -37.6 -9.258579) (width 0.2) (layer "F.Cu") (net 2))
 (segment (start -37.6 -9.258579) (end -38.358579 -8.5) (width 0.2) (layer "F.Cu") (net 2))
 (segment (start -36.5 -19.7) (end -37.6 -18.6) (width 0.2) (layer "F.Cu") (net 2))
 (segment (start -38.358579 -8.5) (end -48 -8.5) (width 0.2) (layer "F.Cu") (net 2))
 (segment (start 71 -16.6) (end 37.475736 -16.6) (width 0.2) (layer "F.Cu") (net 2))
 (segment (start 35.672 -19.7) (end -36.5 -19.7) (width 0.2) (layer "F.Cu") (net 2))
 (segment (start 37.475736 -16.6) (end 37.3 -16.775736) (width 0.2) (layer "F.Cu") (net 2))
 (segment (start -48 -8.5) (end -51.5 -5) (width 0.2) (layer "F.Cu") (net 2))
 (segment (start 37.3 -16.775736) (end 37.3 -18.072) (width 0.2) (layer "F.Cu") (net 2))
 (segment (start 36.7 -17.656) (end 35.256 -19.1) (width 0.2) (layer "F.Cu") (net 4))
 (segment (start 70.999999 -15.999999) (end 37.227208 -16) (width 0.2) (layer "F.Cu") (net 4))
 (segment (start 35.256 -19.1) (end -36.251472 -19.1) (width 0.2) (layer "F.Cu") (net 4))
 (segment (start 37.227208 -16) (end 36.7 -16.527208) (width 0.2) (layer "F.Cu") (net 4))
 (segment (start 73.8 -42.55) (end 73.8 -18.8) (width 0.2) (layer "F.Cu") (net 4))
 (segment (start -37 -18.351472) (end -37 -8.5) (width 0.2) (layer "F.Cu") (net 4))
 (segment (start 36.7 -16.527208) (end 36.7 -17.656) (width 0.2) (layer "F.Cu") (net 4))
 (segment (start -36.251472 -19.1) (end -37 -18.351472) (width 0.2) (layer "F.Cu") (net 4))
 (segment (start -37 -8.5) (end -36.3 -7.8) (width 0.2) (layer "F.Cu") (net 4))
 (segment (start 70.999999 -13.9) (end 36.9 -13.9) (width 0.2) (layer "F.Cu") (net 10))
 (segment (start 75.9 -42.55) (end 75.9 -18.8) (width 0.2) (layer "F.Cu") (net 10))
 (segment (start 36.9 -13.9) (end 36.2 -13.9) (width 0.2) (layer "F.Cu") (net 10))
 (segment (start 35.752 -13.4) (end 35.814 -13.462) (width 0.2) (layer "F.Cu") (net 10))
 (segment (start 36.2 -13.9) (end 35.7 -13.4) (width 0.2) (layer "F.Cu") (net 10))
 (segment (start 35.7 -13.4) (end 35.752 -13.4) (width 0.2) (layer "F.Cu") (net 10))
 (via (at 33.528 -13.462) (size 0.8) (drill 0.4) (layers "F.Cu" "B.Cu") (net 10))
 (via (at 35.814 -13.462) (size 0.8) (drill 0.4) (layers "F.Cu" "B.Cu") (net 10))
 (segment (start 35.814 -13.462) (end 33.528 -13.462) (width 0.2) (layer "B.Cu") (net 10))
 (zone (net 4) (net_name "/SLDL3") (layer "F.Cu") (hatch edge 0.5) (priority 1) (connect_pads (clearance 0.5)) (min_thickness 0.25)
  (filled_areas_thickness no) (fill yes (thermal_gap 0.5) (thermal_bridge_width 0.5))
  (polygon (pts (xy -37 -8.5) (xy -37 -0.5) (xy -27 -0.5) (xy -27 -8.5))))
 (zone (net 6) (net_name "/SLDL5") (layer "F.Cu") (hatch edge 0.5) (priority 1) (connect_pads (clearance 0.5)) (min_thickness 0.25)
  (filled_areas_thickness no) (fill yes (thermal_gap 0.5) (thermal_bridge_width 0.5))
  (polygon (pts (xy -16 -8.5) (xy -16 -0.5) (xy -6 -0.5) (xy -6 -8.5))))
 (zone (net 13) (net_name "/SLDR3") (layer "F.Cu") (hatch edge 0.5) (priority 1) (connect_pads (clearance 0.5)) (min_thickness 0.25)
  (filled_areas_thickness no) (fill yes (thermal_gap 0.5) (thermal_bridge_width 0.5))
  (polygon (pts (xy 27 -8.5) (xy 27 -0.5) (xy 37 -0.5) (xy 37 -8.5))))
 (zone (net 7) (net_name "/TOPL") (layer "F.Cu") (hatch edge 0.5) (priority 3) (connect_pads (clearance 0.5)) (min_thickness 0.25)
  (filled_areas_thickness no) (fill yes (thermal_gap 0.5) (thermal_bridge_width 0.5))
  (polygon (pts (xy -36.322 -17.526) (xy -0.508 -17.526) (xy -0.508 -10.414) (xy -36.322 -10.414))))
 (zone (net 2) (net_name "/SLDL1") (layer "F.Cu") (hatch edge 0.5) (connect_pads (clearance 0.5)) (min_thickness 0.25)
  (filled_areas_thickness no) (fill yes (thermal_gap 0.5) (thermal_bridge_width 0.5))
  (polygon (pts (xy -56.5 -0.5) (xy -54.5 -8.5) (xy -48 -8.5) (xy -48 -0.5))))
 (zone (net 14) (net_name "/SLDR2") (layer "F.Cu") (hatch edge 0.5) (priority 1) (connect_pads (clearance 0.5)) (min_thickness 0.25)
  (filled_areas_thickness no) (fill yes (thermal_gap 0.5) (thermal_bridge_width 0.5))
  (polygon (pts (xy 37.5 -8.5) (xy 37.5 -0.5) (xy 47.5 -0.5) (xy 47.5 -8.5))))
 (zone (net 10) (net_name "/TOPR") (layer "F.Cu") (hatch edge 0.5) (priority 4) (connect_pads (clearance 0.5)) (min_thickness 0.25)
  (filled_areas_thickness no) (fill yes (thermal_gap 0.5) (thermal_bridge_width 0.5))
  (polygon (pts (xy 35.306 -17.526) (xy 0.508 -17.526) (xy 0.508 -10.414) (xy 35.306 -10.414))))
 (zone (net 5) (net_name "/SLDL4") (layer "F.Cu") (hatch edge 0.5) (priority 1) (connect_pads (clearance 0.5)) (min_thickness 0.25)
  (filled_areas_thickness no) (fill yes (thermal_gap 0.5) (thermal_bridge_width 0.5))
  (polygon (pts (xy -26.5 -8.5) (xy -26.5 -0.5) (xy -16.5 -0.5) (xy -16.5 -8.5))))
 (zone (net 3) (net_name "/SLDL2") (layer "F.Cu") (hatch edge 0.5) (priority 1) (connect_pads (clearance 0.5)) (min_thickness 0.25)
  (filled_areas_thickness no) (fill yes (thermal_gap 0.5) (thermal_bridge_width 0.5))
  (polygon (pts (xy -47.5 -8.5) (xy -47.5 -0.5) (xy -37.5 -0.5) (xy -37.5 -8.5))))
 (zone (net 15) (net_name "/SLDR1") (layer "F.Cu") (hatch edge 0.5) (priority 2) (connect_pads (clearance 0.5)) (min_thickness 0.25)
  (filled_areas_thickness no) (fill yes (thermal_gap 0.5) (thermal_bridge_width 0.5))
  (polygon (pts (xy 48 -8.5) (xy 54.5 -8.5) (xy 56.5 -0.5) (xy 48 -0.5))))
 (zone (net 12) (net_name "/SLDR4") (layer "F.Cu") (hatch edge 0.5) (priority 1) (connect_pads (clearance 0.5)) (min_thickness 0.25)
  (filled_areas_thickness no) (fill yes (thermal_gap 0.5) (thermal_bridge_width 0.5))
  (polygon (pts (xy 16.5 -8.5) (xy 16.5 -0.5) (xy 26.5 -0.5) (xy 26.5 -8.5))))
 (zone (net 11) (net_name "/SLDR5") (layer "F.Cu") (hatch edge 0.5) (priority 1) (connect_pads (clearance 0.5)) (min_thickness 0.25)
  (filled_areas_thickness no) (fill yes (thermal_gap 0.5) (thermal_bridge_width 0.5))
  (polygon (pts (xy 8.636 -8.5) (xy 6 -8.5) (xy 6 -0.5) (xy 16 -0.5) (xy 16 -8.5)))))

